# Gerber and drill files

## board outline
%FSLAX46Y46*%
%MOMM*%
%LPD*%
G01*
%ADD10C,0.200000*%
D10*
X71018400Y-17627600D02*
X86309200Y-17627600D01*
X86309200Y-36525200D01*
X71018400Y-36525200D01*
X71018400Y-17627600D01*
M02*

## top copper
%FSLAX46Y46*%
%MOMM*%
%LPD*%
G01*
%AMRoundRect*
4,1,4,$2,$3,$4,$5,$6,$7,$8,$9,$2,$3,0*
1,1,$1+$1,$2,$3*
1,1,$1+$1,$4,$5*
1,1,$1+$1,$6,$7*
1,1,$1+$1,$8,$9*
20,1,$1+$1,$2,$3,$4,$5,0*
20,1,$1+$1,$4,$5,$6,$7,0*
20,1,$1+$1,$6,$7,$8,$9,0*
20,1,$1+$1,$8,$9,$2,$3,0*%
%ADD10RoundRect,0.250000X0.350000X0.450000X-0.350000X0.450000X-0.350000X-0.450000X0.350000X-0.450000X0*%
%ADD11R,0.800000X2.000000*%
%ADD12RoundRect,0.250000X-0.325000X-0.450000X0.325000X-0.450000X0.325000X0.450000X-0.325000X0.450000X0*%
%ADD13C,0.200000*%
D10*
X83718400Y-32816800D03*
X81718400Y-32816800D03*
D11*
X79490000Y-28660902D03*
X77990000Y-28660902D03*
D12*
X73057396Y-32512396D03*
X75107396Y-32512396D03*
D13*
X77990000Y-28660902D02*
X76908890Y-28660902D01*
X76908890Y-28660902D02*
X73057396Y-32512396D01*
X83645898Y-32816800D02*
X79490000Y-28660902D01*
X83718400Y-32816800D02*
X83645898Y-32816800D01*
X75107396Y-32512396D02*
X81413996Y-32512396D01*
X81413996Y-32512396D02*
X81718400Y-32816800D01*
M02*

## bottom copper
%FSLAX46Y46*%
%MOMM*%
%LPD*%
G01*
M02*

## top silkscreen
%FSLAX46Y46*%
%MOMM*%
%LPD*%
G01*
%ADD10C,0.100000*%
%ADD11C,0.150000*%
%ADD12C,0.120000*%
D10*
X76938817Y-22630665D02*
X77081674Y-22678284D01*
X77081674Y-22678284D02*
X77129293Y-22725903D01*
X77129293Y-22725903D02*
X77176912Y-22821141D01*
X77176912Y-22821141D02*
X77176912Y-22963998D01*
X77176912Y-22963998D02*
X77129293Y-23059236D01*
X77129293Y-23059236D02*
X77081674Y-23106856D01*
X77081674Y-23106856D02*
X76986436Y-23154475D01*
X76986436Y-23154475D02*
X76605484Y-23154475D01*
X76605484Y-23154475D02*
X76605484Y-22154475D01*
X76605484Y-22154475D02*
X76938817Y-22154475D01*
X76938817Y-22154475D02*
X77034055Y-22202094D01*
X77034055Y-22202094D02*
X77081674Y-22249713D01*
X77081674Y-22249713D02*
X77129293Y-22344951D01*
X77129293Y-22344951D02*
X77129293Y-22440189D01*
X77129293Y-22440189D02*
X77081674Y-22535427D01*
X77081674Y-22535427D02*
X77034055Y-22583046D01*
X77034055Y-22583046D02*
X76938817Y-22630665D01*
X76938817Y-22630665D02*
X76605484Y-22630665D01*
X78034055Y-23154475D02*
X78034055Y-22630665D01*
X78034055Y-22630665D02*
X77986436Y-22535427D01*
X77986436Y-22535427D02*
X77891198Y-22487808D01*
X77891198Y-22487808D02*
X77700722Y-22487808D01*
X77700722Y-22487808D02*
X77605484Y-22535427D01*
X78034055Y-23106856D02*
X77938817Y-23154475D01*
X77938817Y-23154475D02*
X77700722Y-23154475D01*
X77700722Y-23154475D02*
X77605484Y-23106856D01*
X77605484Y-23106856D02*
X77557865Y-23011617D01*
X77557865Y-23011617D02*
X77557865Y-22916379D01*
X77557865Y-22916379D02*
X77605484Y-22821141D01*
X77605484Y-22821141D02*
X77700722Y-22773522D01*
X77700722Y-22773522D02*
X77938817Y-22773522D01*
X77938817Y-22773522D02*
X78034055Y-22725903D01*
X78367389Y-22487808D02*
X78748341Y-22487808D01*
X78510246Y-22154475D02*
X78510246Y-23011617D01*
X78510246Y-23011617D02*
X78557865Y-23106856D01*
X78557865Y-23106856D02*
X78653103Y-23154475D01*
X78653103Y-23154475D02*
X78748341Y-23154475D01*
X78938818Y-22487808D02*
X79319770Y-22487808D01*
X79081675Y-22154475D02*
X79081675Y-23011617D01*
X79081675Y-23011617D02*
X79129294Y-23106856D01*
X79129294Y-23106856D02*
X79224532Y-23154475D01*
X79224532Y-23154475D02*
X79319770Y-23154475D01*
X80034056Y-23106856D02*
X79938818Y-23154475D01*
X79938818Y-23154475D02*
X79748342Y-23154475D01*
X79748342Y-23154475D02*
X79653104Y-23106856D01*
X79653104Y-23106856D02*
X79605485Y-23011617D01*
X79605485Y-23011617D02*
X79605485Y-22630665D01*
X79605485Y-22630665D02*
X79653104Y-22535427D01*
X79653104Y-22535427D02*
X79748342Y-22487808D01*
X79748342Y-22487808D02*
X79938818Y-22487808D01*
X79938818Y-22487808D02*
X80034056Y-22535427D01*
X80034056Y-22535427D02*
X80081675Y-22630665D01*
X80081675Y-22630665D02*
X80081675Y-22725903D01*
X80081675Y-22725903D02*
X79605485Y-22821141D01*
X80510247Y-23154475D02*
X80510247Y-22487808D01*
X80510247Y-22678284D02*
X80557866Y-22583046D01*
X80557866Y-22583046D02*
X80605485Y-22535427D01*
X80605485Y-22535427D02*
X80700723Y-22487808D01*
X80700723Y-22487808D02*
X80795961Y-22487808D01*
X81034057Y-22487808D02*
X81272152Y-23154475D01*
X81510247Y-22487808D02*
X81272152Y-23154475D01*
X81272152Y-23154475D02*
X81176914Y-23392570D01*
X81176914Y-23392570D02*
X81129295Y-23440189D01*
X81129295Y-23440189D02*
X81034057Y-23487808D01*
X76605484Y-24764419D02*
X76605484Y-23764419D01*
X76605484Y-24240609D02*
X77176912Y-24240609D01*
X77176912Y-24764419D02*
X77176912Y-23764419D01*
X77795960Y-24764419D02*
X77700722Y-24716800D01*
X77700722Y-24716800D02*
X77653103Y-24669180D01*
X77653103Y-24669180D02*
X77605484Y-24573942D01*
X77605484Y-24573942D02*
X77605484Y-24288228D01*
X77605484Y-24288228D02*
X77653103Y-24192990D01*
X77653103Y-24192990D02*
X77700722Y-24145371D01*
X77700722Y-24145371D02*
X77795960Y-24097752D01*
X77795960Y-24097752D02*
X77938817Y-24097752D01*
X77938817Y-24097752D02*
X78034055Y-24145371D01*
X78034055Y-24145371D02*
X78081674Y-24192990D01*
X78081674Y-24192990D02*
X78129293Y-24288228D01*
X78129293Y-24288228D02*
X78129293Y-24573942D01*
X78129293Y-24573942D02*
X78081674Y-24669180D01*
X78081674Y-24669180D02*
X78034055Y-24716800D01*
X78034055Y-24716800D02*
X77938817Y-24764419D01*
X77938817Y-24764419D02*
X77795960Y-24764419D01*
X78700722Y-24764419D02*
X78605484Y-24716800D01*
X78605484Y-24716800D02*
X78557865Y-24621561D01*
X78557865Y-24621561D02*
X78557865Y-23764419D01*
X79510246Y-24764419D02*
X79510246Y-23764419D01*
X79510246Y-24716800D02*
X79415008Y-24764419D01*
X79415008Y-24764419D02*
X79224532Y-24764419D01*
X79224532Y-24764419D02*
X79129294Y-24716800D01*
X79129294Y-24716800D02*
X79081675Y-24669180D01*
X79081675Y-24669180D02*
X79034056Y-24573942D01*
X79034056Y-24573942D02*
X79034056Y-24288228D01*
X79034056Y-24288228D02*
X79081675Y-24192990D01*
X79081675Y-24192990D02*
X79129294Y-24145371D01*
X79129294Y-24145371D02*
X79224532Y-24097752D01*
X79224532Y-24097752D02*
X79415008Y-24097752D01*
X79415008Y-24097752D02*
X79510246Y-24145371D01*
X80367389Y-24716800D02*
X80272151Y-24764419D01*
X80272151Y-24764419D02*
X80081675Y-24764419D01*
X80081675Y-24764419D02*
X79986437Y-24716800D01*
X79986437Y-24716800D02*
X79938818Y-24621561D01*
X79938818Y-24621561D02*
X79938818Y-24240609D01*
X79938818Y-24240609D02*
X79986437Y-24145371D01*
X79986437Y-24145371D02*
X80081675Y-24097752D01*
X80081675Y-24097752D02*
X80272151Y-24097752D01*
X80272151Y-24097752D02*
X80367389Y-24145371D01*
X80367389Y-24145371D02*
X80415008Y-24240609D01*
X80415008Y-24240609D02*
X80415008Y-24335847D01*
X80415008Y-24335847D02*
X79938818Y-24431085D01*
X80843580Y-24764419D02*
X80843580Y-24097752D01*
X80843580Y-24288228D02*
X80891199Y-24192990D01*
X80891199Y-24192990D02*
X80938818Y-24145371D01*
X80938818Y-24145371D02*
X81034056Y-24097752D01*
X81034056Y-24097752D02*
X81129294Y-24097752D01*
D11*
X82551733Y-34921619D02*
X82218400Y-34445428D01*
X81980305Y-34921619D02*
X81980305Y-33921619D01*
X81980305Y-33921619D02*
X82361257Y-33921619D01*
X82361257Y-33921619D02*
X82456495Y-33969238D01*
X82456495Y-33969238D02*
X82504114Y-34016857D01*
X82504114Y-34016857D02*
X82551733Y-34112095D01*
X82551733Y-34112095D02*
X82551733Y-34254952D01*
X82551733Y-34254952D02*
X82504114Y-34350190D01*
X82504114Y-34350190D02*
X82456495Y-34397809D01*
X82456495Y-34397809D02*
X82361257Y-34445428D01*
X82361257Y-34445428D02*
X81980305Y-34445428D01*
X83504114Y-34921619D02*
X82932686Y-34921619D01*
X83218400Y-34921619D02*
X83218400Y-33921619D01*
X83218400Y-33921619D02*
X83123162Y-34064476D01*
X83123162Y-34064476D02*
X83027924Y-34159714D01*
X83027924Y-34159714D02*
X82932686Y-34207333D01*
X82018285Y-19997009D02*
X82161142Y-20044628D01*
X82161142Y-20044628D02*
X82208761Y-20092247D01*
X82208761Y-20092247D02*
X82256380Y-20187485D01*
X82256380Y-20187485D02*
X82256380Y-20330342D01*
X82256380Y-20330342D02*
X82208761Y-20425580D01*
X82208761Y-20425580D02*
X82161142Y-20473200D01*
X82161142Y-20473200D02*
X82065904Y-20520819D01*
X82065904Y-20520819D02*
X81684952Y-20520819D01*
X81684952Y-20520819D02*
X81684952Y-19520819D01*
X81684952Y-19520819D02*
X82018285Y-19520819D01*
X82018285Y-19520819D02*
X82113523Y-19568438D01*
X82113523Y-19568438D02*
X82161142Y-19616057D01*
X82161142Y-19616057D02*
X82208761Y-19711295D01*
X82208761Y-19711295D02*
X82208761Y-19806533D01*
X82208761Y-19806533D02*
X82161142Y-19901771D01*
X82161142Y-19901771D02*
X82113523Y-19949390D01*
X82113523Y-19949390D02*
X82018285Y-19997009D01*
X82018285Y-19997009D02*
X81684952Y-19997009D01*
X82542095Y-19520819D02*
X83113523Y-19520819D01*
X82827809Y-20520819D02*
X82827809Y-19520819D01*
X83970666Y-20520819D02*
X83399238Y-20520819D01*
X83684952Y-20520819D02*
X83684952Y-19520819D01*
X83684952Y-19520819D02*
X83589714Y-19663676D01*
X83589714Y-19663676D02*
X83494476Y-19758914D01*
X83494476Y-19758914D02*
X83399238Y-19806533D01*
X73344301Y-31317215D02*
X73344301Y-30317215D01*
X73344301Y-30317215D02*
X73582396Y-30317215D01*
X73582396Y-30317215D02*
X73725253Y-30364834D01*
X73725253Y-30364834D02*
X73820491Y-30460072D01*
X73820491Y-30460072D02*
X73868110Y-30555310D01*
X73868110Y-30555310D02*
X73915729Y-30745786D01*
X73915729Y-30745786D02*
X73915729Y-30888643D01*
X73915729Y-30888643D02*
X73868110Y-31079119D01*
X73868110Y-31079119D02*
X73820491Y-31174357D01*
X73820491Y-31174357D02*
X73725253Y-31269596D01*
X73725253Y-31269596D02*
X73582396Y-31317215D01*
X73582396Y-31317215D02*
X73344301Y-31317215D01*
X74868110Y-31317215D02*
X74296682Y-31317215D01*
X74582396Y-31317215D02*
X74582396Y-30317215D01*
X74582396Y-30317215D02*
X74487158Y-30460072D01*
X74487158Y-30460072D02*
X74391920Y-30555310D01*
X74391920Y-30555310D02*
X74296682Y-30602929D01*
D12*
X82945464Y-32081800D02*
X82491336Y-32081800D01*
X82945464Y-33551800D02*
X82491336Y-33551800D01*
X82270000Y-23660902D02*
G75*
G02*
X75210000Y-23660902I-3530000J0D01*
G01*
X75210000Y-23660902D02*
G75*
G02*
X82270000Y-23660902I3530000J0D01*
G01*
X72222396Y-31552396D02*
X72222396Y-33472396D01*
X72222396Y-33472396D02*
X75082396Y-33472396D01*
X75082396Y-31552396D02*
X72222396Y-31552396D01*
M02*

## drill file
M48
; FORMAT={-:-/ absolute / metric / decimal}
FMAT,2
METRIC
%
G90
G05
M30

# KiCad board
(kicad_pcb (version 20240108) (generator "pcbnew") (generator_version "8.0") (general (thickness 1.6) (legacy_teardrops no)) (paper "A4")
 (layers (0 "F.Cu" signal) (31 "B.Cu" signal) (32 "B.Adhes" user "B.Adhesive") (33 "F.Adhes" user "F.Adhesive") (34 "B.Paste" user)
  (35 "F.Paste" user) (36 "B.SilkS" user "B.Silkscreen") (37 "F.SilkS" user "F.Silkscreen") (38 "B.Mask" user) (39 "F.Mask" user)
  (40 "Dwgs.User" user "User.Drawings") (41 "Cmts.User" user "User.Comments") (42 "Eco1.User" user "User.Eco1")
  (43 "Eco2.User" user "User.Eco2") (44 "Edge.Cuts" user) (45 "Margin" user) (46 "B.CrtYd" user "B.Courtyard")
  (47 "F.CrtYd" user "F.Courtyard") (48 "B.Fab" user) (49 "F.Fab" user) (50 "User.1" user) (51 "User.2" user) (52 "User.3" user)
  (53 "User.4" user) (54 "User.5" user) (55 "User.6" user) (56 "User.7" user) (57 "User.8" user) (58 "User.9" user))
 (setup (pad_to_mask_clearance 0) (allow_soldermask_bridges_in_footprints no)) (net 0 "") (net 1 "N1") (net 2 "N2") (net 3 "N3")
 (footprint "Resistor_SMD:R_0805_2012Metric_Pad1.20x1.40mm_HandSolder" (layer "F.Cu") (at 82.7184 32.8168 180)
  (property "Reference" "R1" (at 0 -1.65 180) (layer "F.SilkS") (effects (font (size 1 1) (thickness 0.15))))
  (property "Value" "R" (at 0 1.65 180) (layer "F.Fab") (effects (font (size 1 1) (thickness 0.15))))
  (fp_line (start -0.227064 0.735) (end 0.227064 0.735) (stroke (width 0.12) (type solid)) (layer "F.SilkS"))
  (fp_line (start -0.227064 -0.735) (end 0.227064 -0.735) (stroke (width 0.12) (type solid)) (layer "F.SilkS"))
  (pad "1" smd roundrect (at -1 0 180) (size 1.2 1.4) (layers "F.Cu" "F.Paste" "F.Mask") (roundrect_rratio 0.208333) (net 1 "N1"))
  (pad "2" smd roundrect (at 1 0 180) (size 1.2 1.4) (layers "F.Cu" "F.Paste" "F.Mask") (roundrect_rratio 0.208333) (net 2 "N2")))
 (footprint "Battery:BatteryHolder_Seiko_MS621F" (layer "F.Cu") (at 78.74 28.660902 -90)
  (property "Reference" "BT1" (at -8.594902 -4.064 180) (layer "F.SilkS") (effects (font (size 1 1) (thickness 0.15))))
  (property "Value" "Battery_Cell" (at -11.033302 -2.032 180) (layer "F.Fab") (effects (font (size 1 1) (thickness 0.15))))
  (fp_circle (center -5 0) (end -1.47 0) (stroke (width 0.12) (type solid)) (fill none) (layer "F.SilkS"))
  (pad "1" smd rect (at 0 -0.75 270) (size 2 0.8) (layers "F.Cu" "F.Paste" "F.Mask") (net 1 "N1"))
  (pad "2" smd rect (at 0 0.75 270) (size 2 0.8) (layers "F.Cu" "F.Paste" "F.Mask") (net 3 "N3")))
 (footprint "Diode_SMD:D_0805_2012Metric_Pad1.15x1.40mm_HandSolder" (layer "F.Cu") (at 74.082396 32.512396)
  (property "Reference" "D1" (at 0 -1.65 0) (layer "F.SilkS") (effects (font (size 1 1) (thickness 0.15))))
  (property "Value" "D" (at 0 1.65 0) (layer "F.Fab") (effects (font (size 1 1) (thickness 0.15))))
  (fp_line (start -1.86 -0.96) (end -1.86 0.96) (stroke (width 0.12) (type solid)) (layer "F.SilkS"))
  (fp_line (start -1.86 0.96) (end 1 0.96) (stroke (width 0.12) (type solid)) (layer "F.SilkS"))
  (fp_line (start 1 -0.96) (end -1.86 -0.96) (stroke (width 0.12) (type solid)) (layer "F.SilkS"))
  (pad "1" smd roundrect (at -1.025 0) (size 1.15 1.4) (layers "F.Cu" "F.Paste" "F.Mask") (roundrect_rratio 0.217391) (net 3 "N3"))
  (pad "2" smd roundrect (at 1.025 0) (size 1.15 1.4) (layers "F.Cu" "F.Paste" "F.Mask") (roundrect_rratio 0.217391) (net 2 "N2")))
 (gr_rect (start 71.0184 17.6276) (end 86.3092 36.5252) (stroke (width 0.2) (type default)) (fill none) (layer "Edge.Cuts"))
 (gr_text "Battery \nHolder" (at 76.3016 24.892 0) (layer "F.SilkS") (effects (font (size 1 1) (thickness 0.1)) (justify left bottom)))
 (segment (start 77.99 28.660902) (end 76.90889 28.660902) (width 0.2) (layer "F.Cu") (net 3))
 (segment (start 76.90889 28.660902) (end 73.057396 32.512396) (width 0.2) (layer "F.Cu") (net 3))
 (segment (start 83.645898 32.8168) (end 79.49 28.660902) (width 0.2) (layer "F.Cu") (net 1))
 (segment (start 83.7184 32.8168) (end 83.645898 32.8168) (width 0.2) (layer "F.Cu") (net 1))
 (segment (start 75.107396 32.512396) (end 81.413996 32.512396) (width 0.2) (layer "F.Cu") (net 2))
 (segment (start 81.413996 32.512396) (end 81.7184 32.8168) (width 0.2) (layer "F.Cu") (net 2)))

